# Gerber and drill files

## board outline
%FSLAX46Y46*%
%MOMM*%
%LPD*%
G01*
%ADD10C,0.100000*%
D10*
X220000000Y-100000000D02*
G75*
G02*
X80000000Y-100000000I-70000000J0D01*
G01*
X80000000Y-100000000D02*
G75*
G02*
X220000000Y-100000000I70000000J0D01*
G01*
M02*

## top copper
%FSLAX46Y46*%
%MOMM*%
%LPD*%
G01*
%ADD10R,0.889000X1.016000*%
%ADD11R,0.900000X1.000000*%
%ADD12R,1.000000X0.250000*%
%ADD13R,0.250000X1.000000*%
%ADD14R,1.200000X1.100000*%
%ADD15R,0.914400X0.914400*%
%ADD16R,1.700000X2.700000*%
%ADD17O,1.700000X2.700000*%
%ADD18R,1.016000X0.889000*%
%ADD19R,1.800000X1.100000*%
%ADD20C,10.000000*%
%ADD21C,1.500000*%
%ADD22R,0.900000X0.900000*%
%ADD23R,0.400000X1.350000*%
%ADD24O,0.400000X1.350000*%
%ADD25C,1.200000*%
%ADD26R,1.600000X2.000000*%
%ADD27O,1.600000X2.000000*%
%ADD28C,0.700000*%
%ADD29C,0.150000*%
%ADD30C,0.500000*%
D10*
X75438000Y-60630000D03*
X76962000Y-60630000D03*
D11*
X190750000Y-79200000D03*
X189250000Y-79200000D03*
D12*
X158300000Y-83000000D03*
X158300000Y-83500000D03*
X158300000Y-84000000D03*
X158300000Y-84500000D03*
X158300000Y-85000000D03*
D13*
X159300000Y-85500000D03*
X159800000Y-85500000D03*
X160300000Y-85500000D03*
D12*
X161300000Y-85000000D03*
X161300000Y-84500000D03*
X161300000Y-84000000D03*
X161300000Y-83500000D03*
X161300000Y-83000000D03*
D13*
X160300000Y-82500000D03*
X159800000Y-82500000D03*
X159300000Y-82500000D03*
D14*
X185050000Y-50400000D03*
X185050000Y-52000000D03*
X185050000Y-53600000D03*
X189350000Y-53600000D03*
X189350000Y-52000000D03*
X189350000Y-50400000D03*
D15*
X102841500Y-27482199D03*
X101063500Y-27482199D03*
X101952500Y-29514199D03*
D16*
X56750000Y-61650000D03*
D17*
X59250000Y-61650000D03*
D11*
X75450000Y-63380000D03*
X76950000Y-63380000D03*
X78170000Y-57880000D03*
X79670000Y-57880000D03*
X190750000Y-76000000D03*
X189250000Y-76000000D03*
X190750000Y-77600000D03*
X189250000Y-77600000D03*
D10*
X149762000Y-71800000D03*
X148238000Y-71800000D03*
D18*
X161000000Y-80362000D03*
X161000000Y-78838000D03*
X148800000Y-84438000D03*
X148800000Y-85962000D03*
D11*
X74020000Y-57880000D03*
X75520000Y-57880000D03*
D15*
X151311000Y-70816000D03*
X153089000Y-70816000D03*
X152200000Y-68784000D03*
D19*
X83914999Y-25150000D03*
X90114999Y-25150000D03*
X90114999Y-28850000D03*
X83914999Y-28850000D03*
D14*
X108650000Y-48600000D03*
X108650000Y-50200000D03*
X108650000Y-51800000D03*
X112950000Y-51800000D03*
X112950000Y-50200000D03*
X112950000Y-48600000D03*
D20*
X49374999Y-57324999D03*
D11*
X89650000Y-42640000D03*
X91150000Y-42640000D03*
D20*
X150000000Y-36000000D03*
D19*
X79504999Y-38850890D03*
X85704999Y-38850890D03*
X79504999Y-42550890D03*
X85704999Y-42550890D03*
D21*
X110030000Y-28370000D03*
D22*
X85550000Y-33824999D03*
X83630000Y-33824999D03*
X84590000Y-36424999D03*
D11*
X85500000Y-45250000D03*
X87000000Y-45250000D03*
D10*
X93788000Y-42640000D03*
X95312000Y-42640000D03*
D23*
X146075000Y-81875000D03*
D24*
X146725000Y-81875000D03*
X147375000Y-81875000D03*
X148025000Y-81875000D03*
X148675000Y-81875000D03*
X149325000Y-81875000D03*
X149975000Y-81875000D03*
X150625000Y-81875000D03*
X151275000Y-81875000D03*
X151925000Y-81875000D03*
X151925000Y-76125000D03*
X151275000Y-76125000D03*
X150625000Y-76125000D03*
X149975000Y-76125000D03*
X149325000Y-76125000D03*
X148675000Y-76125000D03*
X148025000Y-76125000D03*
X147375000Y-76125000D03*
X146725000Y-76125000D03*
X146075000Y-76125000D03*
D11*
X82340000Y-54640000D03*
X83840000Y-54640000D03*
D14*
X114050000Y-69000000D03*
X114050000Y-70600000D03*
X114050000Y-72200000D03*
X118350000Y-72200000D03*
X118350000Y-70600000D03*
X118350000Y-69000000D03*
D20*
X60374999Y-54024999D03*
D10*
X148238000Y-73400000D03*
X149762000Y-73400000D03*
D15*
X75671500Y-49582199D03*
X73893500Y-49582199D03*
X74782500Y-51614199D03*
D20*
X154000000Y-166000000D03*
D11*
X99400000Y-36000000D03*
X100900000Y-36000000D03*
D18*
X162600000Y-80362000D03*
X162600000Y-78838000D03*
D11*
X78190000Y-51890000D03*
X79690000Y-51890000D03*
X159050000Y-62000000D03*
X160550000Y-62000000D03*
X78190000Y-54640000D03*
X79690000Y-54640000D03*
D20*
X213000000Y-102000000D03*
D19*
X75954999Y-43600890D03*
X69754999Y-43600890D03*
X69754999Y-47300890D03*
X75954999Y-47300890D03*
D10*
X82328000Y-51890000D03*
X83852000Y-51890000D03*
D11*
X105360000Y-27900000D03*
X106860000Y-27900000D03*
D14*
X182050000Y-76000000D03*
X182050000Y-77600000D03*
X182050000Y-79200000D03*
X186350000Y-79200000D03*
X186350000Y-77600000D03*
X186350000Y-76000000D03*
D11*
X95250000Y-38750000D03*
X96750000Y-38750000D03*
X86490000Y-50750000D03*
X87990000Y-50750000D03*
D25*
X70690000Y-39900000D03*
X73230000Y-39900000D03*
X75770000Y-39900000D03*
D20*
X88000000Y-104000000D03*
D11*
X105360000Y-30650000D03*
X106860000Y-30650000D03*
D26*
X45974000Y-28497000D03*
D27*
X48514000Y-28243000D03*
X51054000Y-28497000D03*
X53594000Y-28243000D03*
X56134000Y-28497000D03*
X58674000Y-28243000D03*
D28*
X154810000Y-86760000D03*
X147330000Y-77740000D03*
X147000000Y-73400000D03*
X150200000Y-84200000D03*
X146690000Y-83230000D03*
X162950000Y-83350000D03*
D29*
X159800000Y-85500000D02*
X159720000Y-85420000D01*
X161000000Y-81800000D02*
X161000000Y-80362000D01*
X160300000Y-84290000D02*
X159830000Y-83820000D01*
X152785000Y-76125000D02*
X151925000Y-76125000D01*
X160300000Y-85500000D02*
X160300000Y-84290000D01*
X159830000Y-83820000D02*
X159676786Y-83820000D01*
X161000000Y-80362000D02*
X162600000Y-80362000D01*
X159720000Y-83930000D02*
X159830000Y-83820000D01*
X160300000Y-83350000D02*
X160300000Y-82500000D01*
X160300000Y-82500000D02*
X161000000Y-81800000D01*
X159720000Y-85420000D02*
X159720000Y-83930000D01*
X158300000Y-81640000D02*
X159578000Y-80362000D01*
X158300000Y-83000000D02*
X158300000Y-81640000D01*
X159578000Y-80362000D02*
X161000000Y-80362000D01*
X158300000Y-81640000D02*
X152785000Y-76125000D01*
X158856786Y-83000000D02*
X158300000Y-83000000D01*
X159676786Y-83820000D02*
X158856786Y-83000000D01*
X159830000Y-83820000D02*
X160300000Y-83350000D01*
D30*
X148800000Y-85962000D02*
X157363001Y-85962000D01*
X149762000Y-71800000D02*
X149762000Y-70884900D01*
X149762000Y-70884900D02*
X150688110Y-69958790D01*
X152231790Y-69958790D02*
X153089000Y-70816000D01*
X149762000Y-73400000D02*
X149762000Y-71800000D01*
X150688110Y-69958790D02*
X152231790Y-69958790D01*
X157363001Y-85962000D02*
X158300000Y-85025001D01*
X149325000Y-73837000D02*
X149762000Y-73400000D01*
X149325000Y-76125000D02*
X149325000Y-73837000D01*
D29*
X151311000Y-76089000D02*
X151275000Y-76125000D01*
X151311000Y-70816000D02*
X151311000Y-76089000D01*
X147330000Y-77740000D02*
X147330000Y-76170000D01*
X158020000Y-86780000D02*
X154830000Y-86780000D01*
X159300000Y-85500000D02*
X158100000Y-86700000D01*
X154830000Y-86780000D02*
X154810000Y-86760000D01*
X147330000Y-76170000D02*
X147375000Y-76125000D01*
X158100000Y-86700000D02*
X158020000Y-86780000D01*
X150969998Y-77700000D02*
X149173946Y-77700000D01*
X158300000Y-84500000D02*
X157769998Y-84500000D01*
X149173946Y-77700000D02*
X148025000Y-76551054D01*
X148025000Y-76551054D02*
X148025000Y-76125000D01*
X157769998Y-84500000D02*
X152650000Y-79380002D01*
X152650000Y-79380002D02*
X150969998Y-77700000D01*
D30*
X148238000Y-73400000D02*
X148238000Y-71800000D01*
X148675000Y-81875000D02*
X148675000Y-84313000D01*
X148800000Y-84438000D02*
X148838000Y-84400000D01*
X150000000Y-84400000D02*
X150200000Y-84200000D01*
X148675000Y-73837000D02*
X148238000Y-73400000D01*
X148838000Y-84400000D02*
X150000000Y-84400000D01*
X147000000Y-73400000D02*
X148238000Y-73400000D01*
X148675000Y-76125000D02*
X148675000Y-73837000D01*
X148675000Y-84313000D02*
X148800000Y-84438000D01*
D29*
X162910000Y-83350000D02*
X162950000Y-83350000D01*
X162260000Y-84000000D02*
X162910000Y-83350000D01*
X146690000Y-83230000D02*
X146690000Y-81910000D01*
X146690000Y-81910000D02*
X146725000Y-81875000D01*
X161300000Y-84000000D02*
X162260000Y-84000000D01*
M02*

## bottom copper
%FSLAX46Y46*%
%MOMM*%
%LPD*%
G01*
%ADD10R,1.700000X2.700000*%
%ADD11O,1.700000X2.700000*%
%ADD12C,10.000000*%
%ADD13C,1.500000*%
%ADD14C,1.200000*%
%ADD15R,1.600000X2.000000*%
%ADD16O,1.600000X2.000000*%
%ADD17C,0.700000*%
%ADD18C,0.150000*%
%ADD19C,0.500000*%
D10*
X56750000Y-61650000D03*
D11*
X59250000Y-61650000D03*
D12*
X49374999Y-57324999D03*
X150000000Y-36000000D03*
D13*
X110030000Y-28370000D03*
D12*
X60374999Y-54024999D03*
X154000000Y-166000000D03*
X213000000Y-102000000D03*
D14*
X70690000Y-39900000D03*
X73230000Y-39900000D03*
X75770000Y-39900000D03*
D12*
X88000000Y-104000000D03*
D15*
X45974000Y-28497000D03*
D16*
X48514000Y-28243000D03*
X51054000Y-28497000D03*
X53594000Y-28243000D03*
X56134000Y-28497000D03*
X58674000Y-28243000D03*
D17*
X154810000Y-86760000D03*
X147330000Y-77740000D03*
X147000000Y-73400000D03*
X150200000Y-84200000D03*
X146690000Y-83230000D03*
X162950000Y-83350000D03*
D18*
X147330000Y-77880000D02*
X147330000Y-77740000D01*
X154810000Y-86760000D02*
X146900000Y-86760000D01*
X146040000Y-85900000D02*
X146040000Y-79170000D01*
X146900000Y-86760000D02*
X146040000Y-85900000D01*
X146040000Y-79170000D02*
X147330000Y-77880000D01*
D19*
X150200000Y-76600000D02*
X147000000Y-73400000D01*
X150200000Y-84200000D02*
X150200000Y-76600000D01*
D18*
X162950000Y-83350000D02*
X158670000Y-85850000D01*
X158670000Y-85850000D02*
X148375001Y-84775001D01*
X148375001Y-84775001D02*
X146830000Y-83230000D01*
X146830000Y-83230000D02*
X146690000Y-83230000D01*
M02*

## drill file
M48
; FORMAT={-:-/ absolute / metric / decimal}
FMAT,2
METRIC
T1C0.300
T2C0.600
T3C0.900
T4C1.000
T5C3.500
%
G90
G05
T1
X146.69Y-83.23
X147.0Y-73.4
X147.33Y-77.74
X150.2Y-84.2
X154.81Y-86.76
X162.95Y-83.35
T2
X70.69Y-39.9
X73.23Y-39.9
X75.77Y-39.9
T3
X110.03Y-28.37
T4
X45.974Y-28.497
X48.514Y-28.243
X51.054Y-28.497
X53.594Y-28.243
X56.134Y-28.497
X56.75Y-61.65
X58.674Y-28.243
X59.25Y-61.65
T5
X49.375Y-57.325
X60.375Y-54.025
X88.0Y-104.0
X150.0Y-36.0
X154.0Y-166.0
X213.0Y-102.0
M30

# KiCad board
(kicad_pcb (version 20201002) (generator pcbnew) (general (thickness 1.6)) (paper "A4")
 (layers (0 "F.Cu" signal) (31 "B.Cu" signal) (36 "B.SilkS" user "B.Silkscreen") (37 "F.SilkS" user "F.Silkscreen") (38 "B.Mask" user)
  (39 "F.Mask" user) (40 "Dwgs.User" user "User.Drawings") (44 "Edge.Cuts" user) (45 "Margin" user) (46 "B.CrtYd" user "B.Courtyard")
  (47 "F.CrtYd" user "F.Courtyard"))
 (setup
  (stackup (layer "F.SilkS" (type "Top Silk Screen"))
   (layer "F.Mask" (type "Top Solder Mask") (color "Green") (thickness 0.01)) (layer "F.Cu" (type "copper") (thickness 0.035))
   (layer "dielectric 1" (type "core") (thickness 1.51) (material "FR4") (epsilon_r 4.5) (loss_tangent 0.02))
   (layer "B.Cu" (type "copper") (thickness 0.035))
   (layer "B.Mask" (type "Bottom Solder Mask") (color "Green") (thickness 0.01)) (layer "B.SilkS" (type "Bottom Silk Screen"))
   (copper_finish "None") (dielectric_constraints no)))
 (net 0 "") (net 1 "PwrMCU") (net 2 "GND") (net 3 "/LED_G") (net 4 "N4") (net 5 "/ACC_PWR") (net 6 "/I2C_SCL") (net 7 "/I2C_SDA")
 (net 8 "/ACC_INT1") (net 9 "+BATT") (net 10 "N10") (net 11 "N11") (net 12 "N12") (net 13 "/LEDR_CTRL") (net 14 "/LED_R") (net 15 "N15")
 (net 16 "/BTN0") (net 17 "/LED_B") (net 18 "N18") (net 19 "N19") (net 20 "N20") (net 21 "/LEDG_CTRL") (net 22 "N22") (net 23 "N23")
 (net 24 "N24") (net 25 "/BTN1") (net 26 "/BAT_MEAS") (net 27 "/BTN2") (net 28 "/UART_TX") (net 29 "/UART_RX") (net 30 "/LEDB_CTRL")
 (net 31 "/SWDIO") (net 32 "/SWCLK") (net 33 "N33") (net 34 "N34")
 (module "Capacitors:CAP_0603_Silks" (layer "F.Cu") (at 76.2 60.63)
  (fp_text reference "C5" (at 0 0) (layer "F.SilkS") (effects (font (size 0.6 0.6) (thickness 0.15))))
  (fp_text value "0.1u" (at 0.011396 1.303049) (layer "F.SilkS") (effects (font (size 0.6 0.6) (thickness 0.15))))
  (pad "1" smd rect (at -0.762 0) (size 0.889 1.016) (layers "F.Cu" "F.Paste" "F.Mask") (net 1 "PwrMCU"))
  (pad "2" smd rect (at 0.762 0) (size 0.889 1.016) (layers "F.Cu" "F.Paste" "F.Mask") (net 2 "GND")))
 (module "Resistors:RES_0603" (layer "F.Cu") (at 190 79.2 180)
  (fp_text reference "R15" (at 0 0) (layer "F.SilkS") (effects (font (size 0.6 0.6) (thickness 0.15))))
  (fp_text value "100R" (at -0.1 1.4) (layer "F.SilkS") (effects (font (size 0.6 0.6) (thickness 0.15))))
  (pad "1" smd rect (at -0.75 0 180) (size 0.9 1) (layers "F.Cu" "F.Paste" "F.Mask") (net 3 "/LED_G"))
  (pad "2" smd rect (at 0.75 0 180) (size 0.9 1) (layers "F.Cu" "F.Paste" "F.Mask") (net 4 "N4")))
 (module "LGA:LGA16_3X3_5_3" (layer "F.Cu") (at 159.8 84)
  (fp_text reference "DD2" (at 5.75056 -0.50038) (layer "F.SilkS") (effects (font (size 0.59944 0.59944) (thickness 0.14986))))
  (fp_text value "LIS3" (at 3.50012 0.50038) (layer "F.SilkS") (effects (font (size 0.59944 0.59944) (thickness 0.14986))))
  (pad "1" smd rect (at -1.5 -1) (size 1 0.25) (layers "F.Cu" "F.Paste" "F.Mask") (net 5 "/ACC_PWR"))
  (pad "2" smd rect (at -1.5 -0.5) (size 1 0.25) (layers "F.Cu" "F.Paste" "F.Mask"))
  (pad "3" smd rect (at -1.5 0) (size 1 0.25) (layers "F.Cu" "F.Paste" "F.Mask"))
  (pad "4" smd rect (at -1.5 0.5) (size 1 0.25) (layers "F.Cu" "F.Paste" "F.Mask") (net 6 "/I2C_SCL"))
  (pad "5" smd rect (at -1.5 1) (size 1 0.25) (layers "F.Cu" "F.Paste" "F.Mask") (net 2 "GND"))
  (pad "6" smd rect (at -0.5 1.5 90) (size 1 0.25) (layers "F.Cu" "F.Paste" "F.Mask") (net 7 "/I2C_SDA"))
  (pad "7" smd rect (at 0 1.5 90) (size 1 0.25) (layers "F.Cu" "F.Paste" "F.Mask") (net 5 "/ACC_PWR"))
  (pad "8" smd rect (at 0.5 1.5 90) (size 1 0.25) (layers "F.Cu" "F.Paste" "F.Mask") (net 5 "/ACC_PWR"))
  (pad "9" smd rect (at 1.5 1) (size 1 0.25) (layers "F.Cu" "F.Paste" "F.Mask"))
  (pad "10" smd rect (at 1.5 0.5) (size 1 0.25) (layers "F.Cu" "F.Paste" "F.Mask") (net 2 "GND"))
  (pad "11" smd rect (at 1.5 0) (size 1 0.25) (layers "F.Cu" "F.Paste" "F.Mask") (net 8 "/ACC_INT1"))
  (pad "12" smd rect (at 1.5 -0.5) (size 1 0.25) (layers "F.Cu" "F.Paste" "F.Mask") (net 2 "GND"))
  (pad "13" smd rect (at 1.5 -1) (size 1 0.25) (layers "F.Cu" "F.Paste" "F.Mask"))
  (pad "14" smd rect (at 0.5 -1.5 90) (size 1 0.25) (layers "F.Cu" "F.Paste" "F.Mask") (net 5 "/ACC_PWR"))
  (pad "15" smd rect (at 0 -1.5 90) (size 1 0.25) (layers "F.Cu" "F.Paste" "F.Mask"))
  (pad "16" smd rect (at -0.5 -1.5 90) (size 1 0.25) (layers "F.Cu" "F.Paste" "F.Mask")))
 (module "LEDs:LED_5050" (layer "F.Cu") (at 187.2 52)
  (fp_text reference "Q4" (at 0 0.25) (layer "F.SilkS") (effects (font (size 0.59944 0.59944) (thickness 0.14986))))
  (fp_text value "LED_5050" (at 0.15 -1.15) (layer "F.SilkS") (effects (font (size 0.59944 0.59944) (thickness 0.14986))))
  (pad "1" smd rect (at -2.15 -1.6) (size 1.2 1.1) (layers "F.Cu" "F.Paste" "F.Mask") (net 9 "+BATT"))
  (pad "2" smd rect (at -2.15 0) (size 1.2 1.1) (layers "F.Cu" "F.Paste" "F.Mask") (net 9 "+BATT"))
  (pad "3" smd rect (at -2.15 1.6) (size 1.2 1.1) (layers "F.Cu" "F.Paste" "F.Mask") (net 9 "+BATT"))
  (pad "4" smd rect (at 2.15 1.6) (size 1.2 1.1) (layers "F.Cu" "F.Paste" "F.Mask") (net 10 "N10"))
  (pad "5" smd rect (at 2.15 0) (size 1.2 1.1) (layers "F.Cu" "F.Paste" "F.Mask") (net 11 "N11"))
  (pad "6" smd rect (at 2.15 -1.6) (size 1.2 1.1) (layers "F.Cu" "F.Paste" "F.Mask") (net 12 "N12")))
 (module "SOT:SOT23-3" (layer "F.Cu") (at 101.9525 28.498199)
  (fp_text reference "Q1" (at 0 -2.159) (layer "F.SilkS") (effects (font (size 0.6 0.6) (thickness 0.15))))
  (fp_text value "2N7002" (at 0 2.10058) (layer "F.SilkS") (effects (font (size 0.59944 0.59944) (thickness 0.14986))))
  (pad "1" smd rect (at 0.889 -1.016) (size 0.9144 0.9144) (layers "F.Cu" "F.Paste" "F.Mask") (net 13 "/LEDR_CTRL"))
  (pad "2" smd rect (at -0.889 -1.016) (size 0.9144 0.9144) (layers "F.Cu" "F.Paste" "F.Mask") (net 2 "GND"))
  (pad "3" smd rect (at 0 1.016) (size 0.9144 0.9144) (layers "F.Cu" "F.Paste" "F.Mask") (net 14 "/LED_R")))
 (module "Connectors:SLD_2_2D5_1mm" (layer "F.Cu") (at 58 61.65)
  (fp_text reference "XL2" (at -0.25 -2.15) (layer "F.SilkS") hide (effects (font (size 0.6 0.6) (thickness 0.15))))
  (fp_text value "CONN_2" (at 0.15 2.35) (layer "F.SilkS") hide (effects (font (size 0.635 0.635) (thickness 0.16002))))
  (pad "1" thru_hole rect (at -1.25 0) (size 1.7 2.7) (drill 1) (layers *.Cu *.Mask) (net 2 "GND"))
  (pad "2" thru_hole oval (at 1.25 0) (size 1.7 2.7) (drill 1) (layers *.Cu *.Mask) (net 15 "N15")))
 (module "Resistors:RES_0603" (layer "F.Cu") (at 76.2 63.38)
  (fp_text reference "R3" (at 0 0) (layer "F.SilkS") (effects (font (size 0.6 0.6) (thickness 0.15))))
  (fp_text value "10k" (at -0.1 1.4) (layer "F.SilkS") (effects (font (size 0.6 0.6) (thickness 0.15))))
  (pad "1" smd rect (at -0.75 0) (size 0.9 1) (layers "F.Cu" "F.Paste" "F.Mask") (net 7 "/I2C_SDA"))
  (pad "2" smd rect (at 0.75 0) (size 0.9 1) (layers "F.Cu" "F.Paste" "F.Mask") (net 5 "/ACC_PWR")))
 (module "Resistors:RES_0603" (layer "F.Cu") (at 78.92 57.88)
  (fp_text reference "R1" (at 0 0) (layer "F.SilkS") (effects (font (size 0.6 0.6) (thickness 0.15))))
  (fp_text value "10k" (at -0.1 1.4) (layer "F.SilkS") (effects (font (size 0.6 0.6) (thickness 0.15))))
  (pad "1" smd rect (at -0.75 0) (size 0.9 1) (layers "F.Cu" "F.Paste" "F.Mask") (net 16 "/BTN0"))
  (pad "2" smd rect (at 0.75 0) (size 0.9 1) (layers "F.Cu" "F.Paste" "F.Mask") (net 2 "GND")))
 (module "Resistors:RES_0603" (layer "F.Cu") (at 190 76 180)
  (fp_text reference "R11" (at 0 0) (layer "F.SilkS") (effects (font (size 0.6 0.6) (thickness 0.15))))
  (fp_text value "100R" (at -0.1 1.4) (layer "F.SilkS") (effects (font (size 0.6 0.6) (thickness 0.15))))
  (pad "1" smd rect (at -0.75 0 180) (size 0.9 1) (layers "F.Cu" "F.Paste" "F.Mask") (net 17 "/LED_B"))
  (pad "2" smd rect (at 0.75 0 180) (size 0.9 1) (layers "F.Cu" "F.Paste" "F.Mask") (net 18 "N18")))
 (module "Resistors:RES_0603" (layer "F.Cu") (at 190 77.6 180)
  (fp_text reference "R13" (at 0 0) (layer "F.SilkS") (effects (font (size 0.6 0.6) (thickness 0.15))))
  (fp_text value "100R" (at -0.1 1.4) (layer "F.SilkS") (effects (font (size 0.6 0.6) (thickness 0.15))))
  (pad "1" smd rect (at -0.75 0 180) (size 0.9 1) (layers "F.Cu" "F.Paste" "F.Mask") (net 14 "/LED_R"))
  (pad "2" smd rect (at 0.75 0 180) (size 0.9 1) (layers "F.Cu" "F.Paste" "F.Mask") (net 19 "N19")))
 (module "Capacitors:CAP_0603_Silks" (layer "F.Cu") (at 149 71.8 180)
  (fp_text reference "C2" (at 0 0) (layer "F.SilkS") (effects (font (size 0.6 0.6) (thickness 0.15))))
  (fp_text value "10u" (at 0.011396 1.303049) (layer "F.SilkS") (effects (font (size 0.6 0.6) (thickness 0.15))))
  (pad "1" smd rect (at -0.762 0 180) (size 0.889 1.016) (layers "F.Cu" "F.Paste" "F.Mask") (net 2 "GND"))
  (pad "2" smd rect (at 0.762 0 180) (size 0.889 1.016) (layers "F.Cu" "F.Paste" "F.Mask") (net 1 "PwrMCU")))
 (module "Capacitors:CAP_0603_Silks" (layer "F.Cu") (at 161 79.6 90)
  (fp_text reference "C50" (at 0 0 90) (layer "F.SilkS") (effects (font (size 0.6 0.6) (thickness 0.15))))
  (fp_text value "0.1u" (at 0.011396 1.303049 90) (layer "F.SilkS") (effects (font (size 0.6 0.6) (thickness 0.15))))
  (pad "1" smd rect (at -0.762 0 90) (size 0.889 1.016) (layers "F.Cu" "F.Paste" "F.Mask") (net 5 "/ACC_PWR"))
  (pad "2" smd rect (at 0.762 0 90) (size 0.889 1.016) (layers "F.Cu" "F.Paste" "F.Mask") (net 2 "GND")))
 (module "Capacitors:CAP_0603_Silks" (layer "F.Cu") (at 148.8 85.2 -90)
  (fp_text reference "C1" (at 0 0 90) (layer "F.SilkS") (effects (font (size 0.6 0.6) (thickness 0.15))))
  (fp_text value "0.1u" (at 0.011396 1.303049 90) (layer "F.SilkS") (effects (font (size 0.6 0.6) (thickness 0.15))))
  (pad "1" smd rect (at -0.762 0 270) (size 0.889 1.016) (layers "F.Cu" "F.Paste" "F.Mask") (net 1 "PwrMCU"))
  (pad "2" smd rect (at 0.762 0 270) (size 0.889 1.016) (layers "F.Cu" "F.Paste" "F.Mask") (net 2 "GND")))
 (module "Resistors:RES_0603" (layer "F.Cu") (at 74.77 57.88)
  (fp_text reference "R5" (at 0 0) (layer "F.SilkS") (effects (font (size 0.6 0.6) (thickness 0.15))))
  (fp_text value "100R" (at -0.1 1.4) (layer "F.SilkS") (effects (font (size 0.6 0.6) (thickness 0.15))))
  (pad "1" smd rect (at -0.75 0) (size 0.9 1) (layers "F.Cu" "F.Paste" "F.Mask") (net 17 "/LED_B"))
  (pad "2" smd rect (at 0.75 0) (size 0.9 1) (layers "F.Cu" "F.Paste" "F.Mask") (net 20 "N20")))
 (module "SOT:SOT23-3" (layer "F.Cu") (at 152.2 69.8 180)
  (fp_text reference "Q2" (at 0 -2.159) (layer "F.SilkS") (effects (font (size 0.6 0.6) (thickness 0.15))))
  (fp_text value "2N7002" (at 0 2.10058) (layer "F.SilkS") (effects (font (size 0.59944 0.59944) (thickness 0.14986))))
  (pad "1" smd rect (at 0.889 -1.016 180) (size 0.9144 0.9144) (layers "F.Cu" "F.Paste" "F.Mask") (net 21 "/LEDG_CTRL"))
  (pad "2" smd rect (at -0.889 -1.016 180) (size 0.9144 0.9144) (layers "F.Cu" "F.Paste" "F.Mask") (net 2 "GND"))
  (pad "3" smd rect (at 0 1.016 180) (size 0.9144 0.9144) (layers "F.Cu" "F.Paste" "F.Mask") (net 3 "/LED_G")))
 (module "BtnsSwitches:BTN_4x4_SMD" (layer "F.Cu") (at 87.014999 27)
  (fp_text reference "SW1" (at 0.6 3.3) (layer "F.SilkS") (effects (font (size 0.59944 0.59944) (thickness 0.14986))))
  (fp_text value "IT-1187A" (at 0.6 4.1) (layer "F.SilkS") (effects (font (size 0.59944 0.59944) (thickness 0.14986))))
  (pad "1" smd rect (at -3.1 -1.85) (size 1.8 1.1) (layers "F.Cu" "F.Paste" "F.Mask") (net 1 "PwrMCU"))
  (pad "1" smd rect (at 3.1 -1.85) (size 1.8 1.1) (layers "F.Cu" "F.Paste" "F.Mask") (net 1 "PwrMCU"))
  (pad "2" smd rect (at 3.1 1.85) (size 1.8 1.1) (layers "F.Cu" "F.Paste" "F.Mask") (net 16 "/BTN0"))
  (pad "2" smd rect (at -3.1 1.85) (size 1.8 1.1) (layers "F.Cu" "F.Paste" "F.Mask") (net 16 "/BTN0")))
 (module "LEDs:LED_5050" (layer "F.Cu") (at 110.8 50.2)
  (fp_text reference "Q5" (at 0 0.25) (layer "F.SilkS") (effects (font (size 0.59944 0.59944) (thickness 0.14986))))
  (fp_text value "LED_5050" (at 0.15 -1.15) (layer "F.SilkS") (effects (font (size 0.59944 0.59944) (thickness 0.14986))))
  (pad "1" smd rect (at -2.15 -1.6) (size 1.2 1.1) (layers "F.Cu" "F.Paste" "F.Mask") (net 9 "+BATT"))
  (pad "2" smd rect (at -2.15 0) (size 1.2 1.1) (layers "F.Cu" "F.Paste" "F.Mask") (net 9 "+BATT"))
  (pad "3" smd rect (at -2.15 1.6) (size 1.2 1.1) (layers "F.Cu" "F.Paste" "F.Mask") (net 9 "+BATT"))
  (pad "4" smd rect (at 2.15 1.6) (size 1.2 1.1) (layers "F.Cu" "F.Paste" "F.Mask") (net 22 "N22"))
  (pad "5" smd rect (at 2.15 0) (size 1.2 1.1) (layers "F.Cu" "F.Paste" "F.Mask") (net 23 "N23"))
  (pad "6" smd rect (at 2.15 -1.6) (size 1.2 1.1) (layers "F.Cu" "F.Paste" "F.Mask") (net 20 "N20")))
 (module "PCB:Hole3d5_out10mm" (layer "F.Cu") (at 49.374999 57.324999)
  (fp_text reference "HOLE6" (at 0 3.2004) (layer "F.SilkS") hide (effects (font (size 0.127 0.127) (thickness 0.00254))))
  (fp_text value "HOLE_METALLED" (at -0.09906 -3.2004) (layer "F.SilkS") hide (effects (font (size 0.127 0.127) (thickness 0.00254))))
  (pad "H" thru_hole circle (at 0 0) (size 10 10) (drill 3.5) (layers *.Cu *.Mask) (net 2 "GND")))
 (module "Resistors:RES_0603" (layer "F.Cu") (at 90.4 42.64)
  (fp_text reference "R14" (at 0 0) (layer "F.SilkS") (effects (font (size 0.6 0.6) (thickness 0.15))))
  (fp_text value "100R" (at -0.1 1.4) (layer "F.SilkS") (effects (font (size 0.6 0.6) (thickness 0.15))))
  (pad "1" smd rect (at -0.75 0) (size 0.9 1) (layers "F.Cu" "F.Paste" "F.Mask") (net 3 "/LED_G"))
  (pad "2" smd rect (at 0.75 0) (size 0.9 1) (layers "F.Cu" "F.Paste" "F.Mask") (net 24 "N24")))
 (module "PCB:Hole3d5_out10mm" (layer "F.Cu") (at 150 36)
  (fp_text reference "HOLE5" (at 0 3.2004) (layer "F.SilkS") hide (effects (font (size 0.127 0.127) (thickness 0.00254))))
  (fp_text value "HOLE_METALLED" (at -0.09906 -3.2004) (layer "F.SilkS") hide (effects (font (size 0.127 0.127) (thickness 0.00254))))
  (pad "H" thru_hole circle (at 0 0) (size 10 10) (drill 3.5) (layers *.Cu *.Mask) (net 2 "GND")))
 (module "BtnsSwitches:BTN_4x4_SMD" (layer "F.Cu") (at 82.604999 40.70089)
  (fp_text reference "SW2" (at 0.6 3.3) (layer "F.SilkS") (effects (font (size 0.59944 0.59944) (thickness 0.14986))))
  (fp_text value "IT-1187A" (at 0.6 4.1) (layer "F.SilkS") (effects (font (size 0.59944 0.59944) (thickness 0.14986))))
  (pad "1" smd rect (at -3.1 -1.85) (size 1.8 1.1) (layers "F.Cu" "F.Paste" "F.Mask") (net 1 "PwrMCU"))
  (pad "1" smd rect (at 3.1 -1.85) (size 1.8 1.1) (layers "F.Cu" "F.Paste" "F.Mask") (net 1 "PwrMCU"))
  (pad "2" smd rect (at -3.1 1.85) (size 1.8 1.1) (layers "F.Cu" "F.Paste" "F.Mask") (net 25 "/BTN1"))
  (pad "2" smd rect (at 3.1 1.85) (size 1.8 1.1) (layers "F.Cu" "F.Paste" "F.Mask") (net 25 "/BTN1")))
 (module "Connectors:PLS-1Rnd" (layer "F.Cu") (at 110.03 28.37)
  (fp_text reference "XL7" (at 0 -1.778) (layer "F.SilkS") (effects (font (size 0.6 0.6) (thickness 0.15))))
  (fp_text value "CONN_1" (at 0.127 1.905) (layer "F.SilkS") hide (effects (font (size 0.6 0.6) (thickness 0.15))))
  (pad "1" thru_hole circle (at 0 0) (size 1.5 1.5) (drill 0.9) (layers *.Cu *.Mask) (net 2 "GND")))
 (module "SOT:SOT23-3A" (layer "F.Cu") (at 84.59 35.124999)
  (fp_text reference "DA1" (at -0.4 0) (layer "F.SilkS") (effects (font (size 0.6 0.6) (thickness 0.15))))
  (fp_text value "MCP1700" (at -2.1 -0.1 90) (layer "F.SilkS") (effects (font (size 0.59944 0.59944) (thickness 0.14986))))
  (pad "1" smd rect (at 0.96 -1.3) (size 0.9 0.9) (layers "F.Cu" "F.Paste" "F.Mask") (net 2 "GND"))
  (pad "2" smd rect (at -0.96 -1.3) (size 0.9 0.9) (layers "F.Cu" "F.Paste" "F.Mask") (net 1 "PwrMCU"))
  (pad "3" smd rect (at 0 1.3) (size 0.9 0.9) (layers "F.Cu" "F.Paste" "F.Mask") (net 9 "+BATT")))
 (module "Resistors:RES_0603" (layer "F.Cu") (at 86.25 45.25)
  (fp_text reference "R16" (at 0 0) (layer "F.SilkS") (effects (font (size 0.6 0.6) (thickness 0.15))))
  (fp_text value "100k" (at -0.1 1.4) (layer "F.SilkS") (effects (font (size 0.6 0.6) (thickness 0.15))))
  (pad "1" smd rect (at -0.75 0) (size 0.9 1) (layers "F.Cu" "F.Paste" "F.Mask") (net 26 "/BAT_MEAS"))
  (pad "2" smd rect (at 0.75 0) (size 0.9 1) (layers "F.Cu" "F.Paste" "F.Mask") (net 9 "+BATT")))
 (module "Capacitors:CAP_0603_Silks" (layer "F.Cu") (at 94.55 42.64)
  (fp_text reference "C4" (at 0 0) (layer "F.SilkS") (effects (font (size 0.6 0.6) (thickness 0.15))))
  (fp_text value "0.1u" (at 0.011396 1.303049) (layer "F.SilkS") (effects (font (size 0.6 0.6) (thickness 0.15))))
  (pad "1" smd rect (at -0.762 0) (size 0.889 1.016) (layers "F.Cu" "F.Paste" "F.Mask") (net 9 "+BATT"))
  (pad "2" smd rect (at 0.762 0) (size 0.889 1.016) (layers "F.Cu" "F.Paste" "F.Mask") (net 2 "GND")))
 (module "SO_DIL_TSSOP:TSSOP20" (layer "F.Cu") (at 149 79)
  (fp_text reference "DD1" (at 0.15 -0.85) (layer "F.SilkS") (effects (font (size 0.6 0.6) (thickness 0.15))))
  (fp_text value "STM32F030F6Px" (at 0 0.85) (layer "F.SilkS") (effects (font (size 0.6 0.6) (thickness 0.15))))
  (pad "1" smd rect (at -2.925 2.875) (size 0.4 1.35) (layers "F.Cu" "F.Paste" "F.Mask") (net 2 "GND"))
  (pad "2" smd oval (at -2.275 2.875) (size 0.4 1.35) (layers "F.Cu" "F.Paste" "F.Mask") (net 8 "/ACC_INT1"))
  (pad "3" smd oval (at -1.625 2.875) (size 0.4 1.35) (layers "F.Cu" "F.Paste" "F.Mask") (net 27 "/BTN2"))
  (pad "4" smd oval (at -0.975 2.875) (size 0.4 1.35) (layers "F.Cu" "F.Paste" "F.Mask"))
  (pad "5" smd oval (at -0.325 2.875) (size 0.4 1.35) (layers "F.Cu" "F.Paste" "F.Mask") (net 1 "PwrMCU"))
  (pad "6" smd oval (at 0.325 2.875) (size 0.4 1.35) (layers "F.Cu" "F.Paste" "F.Mask") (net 16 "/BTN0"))
  (pad "7" smd oval (at 0.975 2.875) (size 0.4 1.35) (layers "F.Cu" "F.Paste" "F.Mask") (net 26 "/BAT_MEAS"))
  (pad "8" smd oval (at 1.625 2.875) (size 0.4 1.35) (layers "F.Cu" "F.Paste" "F.Mask") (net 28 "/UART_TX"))
  (pad "9" smd oval (at 2.275 2.875) (size 0.4 1.35) (layers "F.Cu" "F.Paste" "F.Mask") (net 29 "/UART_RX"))
  (pad "10" smd oval (at 2.925 2.875) (size 0.4 1.35) (layers "F.Cu" "F.Paste" "F.Mask") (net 13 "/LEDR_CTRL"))
  (pad "11" smd oval (at 2.925 -2.875) (size 0.4 1.35) (layers "F.Cu" "F.Paste" "F.Mask") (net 5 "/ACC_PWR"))
  (pad "12" smd oval (at 2.275 -2.875) (size 0.4 1.35) (layers "F.Cu" "F.Paste" "F.Mask") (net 21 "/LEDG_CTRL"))
  (pad "13" smd oval (at 1.625 -2.875) (size 0.4 1.35) (layers "F.Cu" "F.Paste" "F.Mask") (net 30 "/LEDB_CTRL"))
  (pad "14" smd oval (at 0.975 -2.875) (size 0.4 1.35) (layers "F.Cu" "F.Paste" "F.Mask") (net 25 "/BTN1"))
  (pad "15" smd oval (at 0.325 -2.875) (size 0.4 1.35) (layers "F.Cu" "F.Paste" "F.Mask") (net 2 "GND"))
  (pad "16" smd oval (at -0.325 -2.875) (size 0.4 1.35) (layers "F.Cu" "F.Paste" "F.Mask") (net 1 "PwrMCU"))
  (pad "17" smd oval (at -0.975 -2.875) (size 0.4 1.35) (layers "F.Cu" "F.Paste" "F.Mask") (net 6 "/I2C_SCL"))
  (pad "18" smd oval (at -1.625 -2.875) (size 0.4 1.35) (layers "F.Cu" "F.Paste" "F.Mask") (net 7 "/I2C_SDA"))
  (pad "19" smd oval (at -2.275 -2.875) (size 0.4 1.35) (layers "F.Cu" "F.Paste" "F.Mask") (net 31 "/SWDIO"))
  (pad "20" smd oval (at -2.925 -2.875) (size 0.4 1.35) (layers "F.Cu" "F.Paste" "F.Mask") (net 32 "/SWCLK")))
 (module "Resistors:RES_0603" (layer "F.Cu") (at 83.09 54.64)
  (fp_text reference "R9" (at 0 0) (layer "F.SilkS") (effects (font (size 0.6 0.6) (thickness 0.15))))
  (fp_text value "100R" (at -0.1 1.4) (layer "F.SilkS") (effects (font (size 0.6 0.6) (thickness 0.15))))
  (pad "1" smd rect (at -0.75 0) (size 0.9 1) (layers "F.Cu" "F.Paste" "F.Mask") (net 3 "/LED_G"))
  (pad "2" smd rect (at 0.75 0) (size 0.9 1) (layers "F.Cu" "F.Paste" "F.Mask") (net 22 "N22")))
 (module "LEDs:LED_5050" (layer "F.Cu") (at 116.2 70.6)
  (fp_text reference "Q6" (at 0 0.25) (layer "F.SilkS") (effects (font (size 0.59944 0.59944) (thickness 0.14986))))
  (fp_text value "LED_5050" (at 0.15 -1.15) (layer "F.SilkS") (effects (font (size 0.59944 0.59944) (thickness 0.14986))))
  (pad "1" smd rect (at -2.15 -1.6) (size 1.2 1.1) (layers "F.Cu" "F.Paste" "F.Mask") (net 9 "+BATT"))
  (pad "2" smd rect (at -2.15 0) (size 1.2 1.1) (layers "F.Cu" "F.Paste" "F.Mask") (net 9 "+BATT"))
  (pad "3" smd rect (at -2.15 1.6) (size 1.2 1.1) (layers "F.Cu" "F.Paste" "F.Mask") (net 9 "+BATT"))
  (pad "4" smd rect (at 2.15 1.6) (size 1.2 1.1) (layers "F.Cu" "F.Paste" "F.Mask") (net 24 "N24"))
  (pad "5" smd rect (at 2.15 0) (size 1.2 1.1) (layers "F.Cu" "F.Paste" "F.Mask") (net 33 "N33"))
  (pad "6" smd rect (at 2.15 -1.6) (size 1.2 1.1) (layers "F.Cu" "F.Paste" "F.Mask") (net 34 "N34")))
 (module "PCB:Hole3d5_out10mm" (layer "F.Cu") (at 60.374999 54.024999)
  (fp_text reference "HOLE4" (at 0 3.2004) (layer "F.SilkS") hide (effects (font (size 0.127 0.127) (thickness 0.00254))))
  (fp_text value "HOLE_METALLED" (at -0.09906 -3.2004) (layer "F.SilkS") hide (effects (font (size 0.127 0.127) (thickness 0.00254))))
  (pad "H" thru_hole circle (at 0 0) (size 10 10) (drill 3.5) (layers *.Cu *.Mask) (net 2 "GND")))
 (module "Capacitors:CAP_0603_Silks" (layer "F.Cu") (at 149 73.4)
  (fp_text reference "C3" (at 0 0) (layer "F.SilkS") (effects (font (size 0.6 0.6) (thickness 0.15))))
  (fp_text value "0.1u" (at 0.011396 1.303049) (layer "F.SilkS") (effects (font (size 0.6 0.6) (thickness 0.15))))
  (pad "1" smd rect (at -0.762 0) (size 0.889 1.016) (layers "F.Cu" "F.Paste" "F.Mask") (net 1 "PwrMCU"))
  (pad "2" smd rect (at 0.762 0) (size 0.889 1.016) (layers "F.Cu" "F.Paste" "F.Mask") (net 2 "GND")))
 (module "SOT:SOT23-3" (layer "F.Cu") (at 74.7825 50.598199)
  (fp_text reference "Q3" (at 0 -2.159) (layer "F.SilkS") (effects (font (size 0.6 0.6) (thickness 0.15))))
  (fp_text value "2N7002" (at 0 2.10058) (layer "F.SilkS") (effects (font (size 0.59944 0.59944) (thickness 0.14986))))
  (pad "1" smd rect (at 0.889 -1.016) (size 0.9144 0.9144) (layers "F.Cu" "F.Paste" "F.Mask") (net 30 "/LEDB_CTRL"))
  (pad "2" smd rect (at -0.889 -1.016) (size 0.9144 0.9144) (layers "F.Cu" "F.Paste" "F.Mask") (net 2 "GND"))
  (pad "3" smd rect (at 0 1.016) (size 0.9144 0.9144) (layers "F.Cu" "F.Paste" "F.Mask") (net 17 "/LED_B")))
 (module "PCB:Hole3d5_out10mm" (layer "F.Cu") (at 154 166)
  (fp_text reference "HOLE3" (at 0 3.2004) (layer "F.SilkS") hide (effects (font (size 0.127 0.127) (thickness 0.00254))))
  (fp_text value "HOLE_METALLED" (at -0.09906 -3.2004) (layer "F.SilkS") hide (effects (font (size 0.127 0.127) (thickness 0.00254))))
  (pad "H" thru_hole circle (at 0 0) (size 10 10) (drill 3.5) (layers *.Cu *.Mask) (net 2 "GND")))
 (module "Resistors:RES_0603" (layer "F.Cu") (at 100.15 36)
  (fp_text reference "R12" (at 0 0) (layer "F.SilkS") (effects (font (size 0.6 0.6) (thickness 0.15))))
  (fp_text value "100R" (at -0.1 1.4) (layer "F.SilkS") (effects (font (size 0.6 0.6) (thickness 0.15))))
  (pad "1" smd rect (at -0.75 0) (size 0.9 1) (layers "F.Cu" "F.Paste" "F.Mask") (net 14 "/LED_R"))
  (pad "2" smd rect (at 0.75 0) (size 0.9 1) (layers "F.Cu" "F.Paste" "F.Mask") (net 33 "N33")))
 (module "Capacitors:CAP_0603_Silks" (layer "F.Cu") (at 162.6 79.6 90)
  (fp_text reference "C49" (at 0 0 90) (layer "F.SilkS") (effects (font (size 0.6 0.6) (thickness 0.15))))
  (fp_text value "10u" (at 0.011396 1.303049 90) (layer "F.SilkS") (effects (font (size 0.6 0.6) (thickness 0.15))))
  (pad "1" smd rect (at -0.762 0 90) (size 0.889 1.016) (layers "F.Cu" "F.Paste" "F.Mask") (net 5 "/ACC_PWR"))
  (pad "2" smd rect (at 0.762 0 90) (size 0.889 1.016) (layers "F.Cu" "F.Paste" "F.Mask") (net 2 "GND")))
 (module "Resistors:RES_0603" (layer "F.Cu") (at 78.94 51.89)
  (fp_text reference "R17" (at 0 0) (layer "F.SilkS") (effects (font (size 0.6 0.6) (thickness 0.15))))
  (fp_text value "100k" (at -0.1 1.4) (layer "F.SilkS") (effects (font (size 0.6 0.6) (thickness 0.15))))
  (pad "1" smd rect (at -0.75 0) (size 0.9 1) (layers "F.Cu" "F.Paste" "F.Mask") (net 2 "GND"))
  (pad "2" smd rect (at 0.75 0) (size 0.9 1) (layers "F.Cu" "F.Paste" "F.Mask") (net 26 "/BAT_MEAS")))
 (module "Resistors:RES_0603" (layer "F.Cu") (at 159.8 62)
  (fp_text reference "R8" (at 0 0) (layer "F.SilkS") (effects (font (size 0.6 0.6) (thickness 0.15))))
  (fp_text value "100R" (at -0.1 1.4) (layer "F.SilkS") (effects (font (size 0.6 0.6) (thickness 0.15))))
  (pad "1" smd rect (at -0.75 0) (size 0.9 1) (layers "F.Cu" "F.Paste" "F.Mask") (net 3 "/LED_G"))
  (pad "2" smd rect (at 0.75 0) (size 0.9 1) (layers "F.Cu" "F.Paste" "F.Mask") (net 10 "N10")))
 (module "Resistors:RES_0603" (layer "F.Cu") (at 78.94 54.64)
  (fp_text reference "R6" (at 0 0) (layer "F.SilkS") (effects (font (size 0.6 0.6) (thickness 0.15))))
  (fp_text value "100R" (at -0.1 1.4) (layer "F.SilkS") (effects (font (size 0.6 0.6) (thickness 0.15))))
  (pad "1" smd rect (at -0.75 0) (size 0.9 1) (layers "F.Cu" "F.Paste" "F.Mask") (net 14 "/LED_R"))
  (pad "2" smd rect (at 0.75 0) (size 0.9 1) (layers "F.Cu" "F.Paste" "F.Mask") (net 11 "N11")))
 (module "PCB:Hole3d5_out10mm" (layer "F.Cu") (at 213 102)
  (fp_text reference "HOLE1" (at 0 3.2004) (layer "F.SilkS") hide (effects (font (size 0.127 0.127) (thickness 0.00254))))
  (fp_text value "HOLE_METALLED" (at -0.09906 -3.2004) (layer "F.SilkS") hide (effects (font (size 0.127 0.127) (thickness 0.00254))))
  (pad "H" thru_hole circle (at 0 0) (size 10 10) (drill 3.5) (layers *.Cu *.Mask) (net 2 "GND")))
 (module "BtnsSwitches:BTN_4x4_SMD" (layer "F.Cu") (at 72.854999 45.45089)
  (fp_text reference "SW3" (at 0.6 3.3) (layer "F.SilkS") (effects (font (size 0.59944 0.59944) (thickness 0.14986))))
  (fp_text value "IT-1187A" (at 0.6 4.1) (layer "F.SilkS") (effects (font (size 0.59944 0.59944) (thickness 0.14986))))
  (pad "1" smd rect (at 3.1 -1.85) (size 1.8 1.1) (layers "F.Cu" "F.Paste" "F.Mask") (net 1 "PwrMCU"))
  (pad "1" smd rect (at -3.1 -1.85) (size 1.8 1.1) (layers "F.Cu" "F.Paste" "F.Mask") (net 1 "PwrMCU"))
  (pad "2" smd rect (at -3.1 1.85) (size 1.8 1.1) (layers "F.Cu" "F.Paste" "F.Mask") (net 27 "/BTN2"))
  (pad "2" smd rect (at 3.1 1.85) (size 1.8 1.1) (layers "F.Cu" "F.Paste" "F.Mask") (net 27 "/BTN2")))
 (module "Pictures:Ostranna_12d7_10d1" (layer "F.Cu") (at 50.578897 35.505602)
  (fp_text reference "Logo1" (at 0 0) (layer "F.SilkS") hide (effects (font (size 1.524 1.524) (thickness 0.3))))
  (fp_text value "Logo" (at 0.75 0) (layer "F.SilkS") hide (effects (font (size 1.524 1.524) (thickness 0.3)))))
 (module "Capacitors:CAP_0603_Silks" (layer "F.Cu") (at 83.09 51.89)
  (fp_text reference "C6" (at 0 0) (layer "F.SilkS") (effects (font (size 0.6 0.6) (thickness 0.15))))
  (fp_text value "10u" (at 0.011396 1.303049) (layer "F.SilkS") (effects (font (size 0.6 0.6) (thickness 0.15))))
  (pad "1" smd rect (at -0.762 0) (size 0.889 1.016) (layers "F.Cu" "F.Paste" "F.Mask") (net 2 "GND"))
  (pad "2" smd rect (at 0.762 0) (size 0.889 1.016) (layers "F.Cu" "F.Paste" "F.Mask") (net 9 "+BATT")))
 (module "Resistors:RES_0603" (layer "F.Cu") (at 106.11 27.9)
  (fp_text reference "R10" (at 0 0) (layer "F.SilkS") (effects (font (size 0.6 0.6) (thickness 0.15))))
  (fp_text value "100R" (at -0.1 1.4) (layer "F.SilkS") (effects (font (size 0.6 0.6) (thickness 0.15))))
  (pad "1" smd rect (at -0.75 0) (size 0.9 1) (layers "F.Cu" "F.Paste" "F.Mask") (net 17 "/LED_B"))
  (pad "2" smd rect (at 0.75 0) (size 0.9 1) (layers "F.Cu" "F.Paste" "F.Mask") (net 34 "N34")))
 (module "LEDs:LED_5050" (layer "F.Cu") (at 184.2 77.6)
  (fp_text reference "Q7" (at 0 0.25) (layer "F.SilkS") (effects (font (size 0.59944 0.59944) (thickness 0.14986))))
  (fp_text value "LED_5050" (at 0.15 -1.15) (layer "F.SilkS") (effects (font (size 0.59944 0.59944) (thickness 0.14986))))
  (pad "1" smd rect (at -2.15 -1.6) (size 1.2 1.1) (layers "F.Cu" "F.Paste" "F.Mask") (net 9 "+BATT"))
  (pad "2" smd rect (at -2.15 0) (size 1.2 1.1) (layers "F.Cu" "F.Paste" "F.Mask") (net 9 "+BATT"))
  (pad "3" smd rect (at -2.15 1.6) (size 1.2 1.1) (layers "F.Cu" "F.Paste" "F.Mask") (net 9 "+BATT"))
  (pad "4" smd rect (at 2.15 1.6) (size 1.2 1.1) (layers "F.Cu" "F.Paste" "F.Mask") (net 4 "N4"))
  (pad "5" smd rect (at 2.15 0) (size 1.2 1.1) (layers "F.Cu" "F.Paste" "F.Mask") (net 19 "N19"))
  (pad "6" smd rect (at 2.15 -1.6) (size 1.2 1.1) (layers "F.Cu" "F.Paste" "F.Mask") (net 18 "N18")))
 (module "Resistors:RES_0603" (layer "F.Cu") (at 96 38.75)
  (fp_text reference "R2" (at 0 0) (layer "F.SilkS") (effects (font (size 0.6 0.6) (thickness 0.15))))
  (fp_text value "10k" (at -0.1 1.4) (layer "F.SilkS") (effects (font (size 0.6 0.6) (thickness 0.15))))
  (pad "1" smd rect (at -0.75 0) (size 0.9 1) (layers "F.Cu" "F.Paste" "F.Mask") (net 5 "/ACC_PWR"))
  (pad "2" smd rect (at 0.75 0) (size 0.9 1) (layers "F.Cu" "F.Paste" "F.Mask") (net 6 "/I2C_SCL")))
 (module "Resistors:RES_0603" (layer "F.Cu") (at 87.24 50.75)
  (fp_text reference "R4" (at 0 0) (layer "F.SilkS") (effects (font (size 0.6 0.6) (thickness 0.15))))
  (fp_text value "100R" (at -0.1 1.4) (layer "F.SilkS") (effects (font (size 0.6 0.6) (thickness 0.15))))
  (pad "1" smd rect (at -0.75 0) (size 0.9 1) (layers "F.Cu" "F.Paste" "F.Mask") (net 17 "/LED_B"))
  (pad "2" smd rect (at 0.75 0) (size 0.9 1) (layers "F.Cu" "F.Paste" "F.Mask") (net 12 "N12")))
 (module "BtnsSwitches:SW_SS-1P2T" (layer "F.Cu") (at 73.23 39.9)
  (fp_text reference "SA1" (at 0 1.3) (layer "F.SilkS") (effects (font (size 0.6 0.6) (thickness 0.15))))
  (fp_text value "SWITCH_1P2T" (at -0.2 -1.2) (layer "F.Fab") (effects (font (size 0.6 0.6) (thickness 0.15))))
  (pad "1" thru_hole circle (at -2.54 0) (size 1.2 1.2) (drill 0.6) (layers *.Cu *.Mask) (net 9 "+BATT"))
  (pad "2" thru_hole circle (at 0 0) (size 1.2 1.2) (drill 0.6) (layers *.Cu *.Mask) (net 15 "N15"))
  (pad "3" thru_hole circle (at 2.54 0) (size 1.2 1.2) (drill 0.6) (layers *.Cu *.Mask)))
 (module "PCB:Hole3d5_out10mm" (layer "F.Cu") (at 88 104)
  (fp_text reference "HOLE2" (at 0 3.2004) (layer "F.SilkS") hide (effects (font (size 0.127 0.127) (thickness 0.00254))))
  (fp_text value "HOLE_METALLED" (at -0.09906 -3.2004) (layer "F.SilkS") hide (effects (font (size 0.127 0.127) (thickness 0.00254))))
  (pad "H" thru_hole circle (at 0 0) (size 10 10) (drill 3.5) (layers *.Cu *.Mask) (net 2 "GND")))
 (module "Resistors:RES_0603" (layer "F.Cu") (at 106.11 30.65)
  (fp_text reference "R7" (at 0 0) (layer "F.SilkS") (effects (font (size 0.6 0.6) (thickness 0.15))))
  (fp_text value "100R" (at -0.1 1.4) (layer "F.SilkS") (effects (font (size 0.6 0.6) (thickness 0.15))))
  (pad "1" smd rect (at -0.75 0) (size 0.9 1) (layers "F.Cu" "F.Paste" "F.Mask") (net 14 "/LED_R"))
  (pad "2" smd rect (at 0.75 0) (size 0.9 1) (layers "F.Cu" "F.Paste" "F.Mask") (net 23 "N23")))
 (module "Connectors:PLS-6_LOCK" (layer "F.Cu") (at 45.974 28.37)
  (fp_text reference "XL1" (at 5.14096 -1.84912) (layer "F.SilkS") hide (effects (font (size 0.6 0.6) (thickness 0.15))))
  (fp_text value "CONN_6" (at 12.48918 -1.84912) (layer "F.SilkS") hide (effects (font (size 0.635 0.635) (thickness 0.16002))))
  (pad "1" thru_hole rect (at 0 0.127) (size 1.6 2) (drill 1) (layers *.Cu *.Mask) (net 1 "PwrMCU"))
  (pad "2" thru_hole oval (at 2.54 -0.127) (size 1.6 2) (drill 1) (layers *.Cu *.Mask) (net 32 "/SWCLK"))
  (pad "3" thru_hole oval (at 5.08 0.127) (size 1.6 2) (drill 1) (layers *.Cu *.Mask) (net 2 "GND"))
  (pad "4" thru_hole oval (at 7.62 -0.127) (size 1.6 2) (drill 1) (layers *.Cu *.Mask) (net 31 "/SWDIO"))
  (pad "5" thru_hole oval (at 10.16 0.127) (size 1.6 2) (drill 1) (layers *.Cu *.Mask) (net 28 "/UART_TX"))
  (pad "6" thru_hole oval (at 12.7 -0.127) (size 1.6 2) (drill 1) (layers *.Cu *.Mask) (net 29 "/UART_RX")))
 (gr_circle (center 150 100) (end 220 100) (layer "Edge.Cuts") (width 0.1))
 (segment (start 159.8 85.5) (end 159.72 85.42) (width 0.15) (layer "F.Cu") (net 5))
 (segment (start 161 81.8) (end 161 80.362) (width 0.15) (layer "F.Cu") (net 5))
 (segment (start 160.3 84.29) (end 159.83 83.82) (width 0.15) (layer "F.Cu") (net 5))
 (segment (start 152.785 76.125) (end 151.925 76.125) (width 0.15) (layer "F.Cu") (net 5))
 (segment (start 160.3 85.5) (end 160.3 84.29) (width 0.15) (layer "F.Cu") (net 5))
 (segment (start 159.83 83.82) (end 159.676786 83.82) (width 0.15) (layer "F.Cu") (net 5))
 (segment (start 161 80.362) (end 162.6 80.362) (width 0.15) (layer "F.Cu") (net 5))
 (segment (start 159.72 83.93) (end 159.83 83.82) (width 0.15) (layer "F.Cu") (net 5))
 (segment (start 160.3 83.35) (end 160.3 82.5) (width 0.15) (layer "F.Cu") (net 5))
 (segment (start 160.3 82.5) (end 161 81.8) (width 0.15) (layer "F.Cu") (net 5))
 (segment (start 159.72 85.42) (end 159.72 83.93) (width 0.15) (layer "F.Cu") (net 5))
 (segment (start 158.3 81.64) (end 159.578 80.362) (width 0.15) (layer "F.Cu") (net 5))
 (segment (start 158.3 83) (end 158.3 81.64) (width 0.15) (layer "F.Cu") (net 5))
 (segment (start 159.578 80.362) (end 161 80.362) (width 0.15) (layer "F.Cu") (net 5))
 (segment (start 158.3 81.64) (end 152.785 76.125) (width 0.15) (layer "F.Cu") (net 5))
 (segment (start 158.856786 83) (end 158.3 83) (width 0.15) (layer "F.Cu") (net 5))
 (segment (start 159.676786 83.82) (end 158.856786 83) (width 0.15) (layer "F.Cu") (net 5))
 (segment (start 159.83 83.82) (end 160.3 83.35) (width 0.15) (layer "F.Cu") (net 5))
 (segment (start 148.8 85.962) (end 157.363001 85.962) (width 0.5) (layer "F.Cu") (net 2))
 (segment (start 149.762 71.8) (end 149.762 70.8849) (width 0.5) (layer "F.Cu") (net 2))
 (segment (start 149.762 70.8849) (end 150.68811 69.95879) (width 0.5) (layer "F.Cu") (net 2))
 (segment (start 152.23179 69.95879) (end 153.089 70.816) (width 0.5) (layer "F.Cu") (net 2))
 (segment (start 149.762 73.4) (end 149.762 71.8) (width 0.5) (layer "F.Cu") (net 2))
 (segment (start 150.68811 69.95879) (end 152.23179 69.95879) (width 0.5) (layer "F.Cu") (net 2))
 (segment (start 157.363001 85.962) (end 158.3 85.025001) (width 0.5) (layer "F.Cu") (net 2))
 (segment (start 149.325 73.837) (end 149.762 73.4) (width 0.5) (layer "F.Cu") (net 2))
 (segment (start 149.325 76.125) (end 149.325 73.837) (width 0.5) (layer "F.Cu") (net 2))
 (segment (start 151.311 76.089) (end 151.275 76.125) (width 0.15) (layer "F.Cu") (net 21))
 (segment (start 151.311 70.816) (end 151.311 76.089) (width 0.15) (layer "F.Cu") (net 21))
 (segment (start 147.33 77.74) (end 147.33 76.17) (width 0.15) (layer "F.Cu") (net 7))
 (segment (start 158.02 86.78) (end 154.83 86.78) (width 0.15) (layer "F.Cu") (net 7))
 (segment (start 159.3 85.5) (end 158.1 86.7) (width 0.15) (layer "F.Cu") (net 7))
 (segment (start 154.83 86.78) (end 154.81 86.76) (width 0.15) (layer "F.Cu") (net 7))
 (segment (start 147.33 76.17) (end 147.375 76.125) (width 0.15) (layer "F.Cu") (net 7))
 (segment (start 158.1 86.7) (end 158.02 86.78) (width 0.15) (layer "F.Cu") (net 7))
 (via (at 154.81 86.76) (size 0.7) (drill 0.3) (layers "F.Cu" "B.Cu") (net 7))
 (via (at 147.33 77.74) (size 0.7) (drill 0.3) (layers "F.Cu" "B.Cu") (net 7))
 (segment (start 147.33 77.88) (end 147.33 77.74) (width 0.15) (layer "B.Cu") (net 7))
 (segment (start 154.81 86.76) (end 146.9 86.76) (width 0.15) (layer "B.Cu") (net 7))
 (segment (start 146.04 85.9) (end 146.04 79.17) (width 0.15) (layer "B.Cu") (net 7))
 (segment (start 146.9 86.76) (end 146.04 85.9) (width 0.15) (layer "B.Cu") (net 7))
 (segment (start 146.04 79.17) (end 147.33 77.88) (width 0.15) (layer "B.Cu") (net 7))
 (segment (start 150.969998 77.7) (end 149.173946 77.7) (width 0.15) (layer "F.Cu") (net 6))
 (segment (start 158.3 84.5) (end 157.769998 84.5) (width 0.15) (layer "F.Cu") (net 6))
 (segment (start 149.173946 77.7) (end 148.025 76.551054) (width 0.15) (layer "F.Cu") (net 6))
 (segment (start 148.025 76.551054) (end 148.025 76.125) (width 0.15) (layer "F.Cu") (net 6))
 (segment (start 157.769998 84.5) (end 152.65 79.380002) (width 0.15) (layer "F.Cu") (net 6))
 (segment (start 152.65 79.380002) (end 150.969998 77.7) (width 0.15) (layer "F.Cu") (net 6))
 (segment (start 148.238 73.4) (end 148.238 71.8) (width 0.5) (layer "F.Cu") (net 1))
 (segment (start 148.675 81.875) (end 148.675 84.313) (width 0.5) (layer "F.Cu") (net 1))
 (segment (start 148.8 84.438) (end 148.838 84.4) (width 0.5) (layer "F.Cu") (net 1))
 (segment (start 150 84.4) (end 150.2 84.2) (width 0.5) (layer "F.Cu") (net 1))
 (segment (start 148.675 73.837) (end 148.238 73.4) (width 0.5) (layer "F.Cu") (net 1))
 (segment (start 148.838 84.4) (end 150 84.4) (width 0.5) (layer "F.Cu") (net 1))
 (segment (start 147 73.4) (end 148.238 73.4) (width 0.5) (layer "F.Cu") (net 1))
 (segment (start 148.675 76.125) (end 148.675 73.837) (width 0.5) (layer "F.Cu") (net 1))
 (segment (start 148.675 84.313) (end 148.8 84.438) (width 0.5) (layer "F.Cu") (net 1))
 (via (at 147 73.4) (size 0.7) (drill 0.3) (layers "F.Cu" "B.Cu") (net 1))
 (via (at 150.2 84.2) (size 0.7) (drill 0.3) (layers "F.Cu" "B.Cu") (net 1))
 (segment (start 150.2 76.6) (end 147 73.4) (width 0.5) (layer "B.Cu") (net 1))
 (segment (start 150.2 84.2) (end 150.2 76.6) (width 0.5) (layer "B.Cu") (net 1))
 (segment (start 162.91 83.35) (end 162.95 83.35) (width 0.15) (layer "F.Cu") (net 8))
 (segment (start 162.26 84) (end 162.91 83.35) (width 0.15) (layer "F.Cu") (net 8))
 (segment (start 146.69 83.23) (end 146.69 81.91) (width 0.15) (layer "F.Cu") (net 8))
 (segment (start 146.69 81.91) (end 146.725 81.875) (width 0.15) (layer "F.Cu") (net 8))
 (segment (start 161.3 84) (end 162.26 84) (width 0.15) (layer "F.Cu") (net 8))
 (via (at 146.69 83.23) (size 0.7) (drill 0.3) (layers "F.Cu" "B.Cu") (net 8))
 (via (at 162.95 83.35) (size 0.7) (drill 0.3) (layers "F.Cu" "B.Cu") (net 8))
 (segment (start 162.95 83.35) (end 158.67 85.85) (width 0.15) (layer "B.Cu") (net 8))
 (segment (start 158.67 85.85) (end 148.375001 84.775001) (width 0.15) (layer "B.Cu") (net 8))
 (segment (start 148.375001 84.775001) (end 146.83 83.23) (width 0.15) (layer "B.Cu") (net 8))
 (segment (start 146.83 83.23) (end 146.69 83.23) (width 0.15) (layer "B.Cu") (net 8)))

